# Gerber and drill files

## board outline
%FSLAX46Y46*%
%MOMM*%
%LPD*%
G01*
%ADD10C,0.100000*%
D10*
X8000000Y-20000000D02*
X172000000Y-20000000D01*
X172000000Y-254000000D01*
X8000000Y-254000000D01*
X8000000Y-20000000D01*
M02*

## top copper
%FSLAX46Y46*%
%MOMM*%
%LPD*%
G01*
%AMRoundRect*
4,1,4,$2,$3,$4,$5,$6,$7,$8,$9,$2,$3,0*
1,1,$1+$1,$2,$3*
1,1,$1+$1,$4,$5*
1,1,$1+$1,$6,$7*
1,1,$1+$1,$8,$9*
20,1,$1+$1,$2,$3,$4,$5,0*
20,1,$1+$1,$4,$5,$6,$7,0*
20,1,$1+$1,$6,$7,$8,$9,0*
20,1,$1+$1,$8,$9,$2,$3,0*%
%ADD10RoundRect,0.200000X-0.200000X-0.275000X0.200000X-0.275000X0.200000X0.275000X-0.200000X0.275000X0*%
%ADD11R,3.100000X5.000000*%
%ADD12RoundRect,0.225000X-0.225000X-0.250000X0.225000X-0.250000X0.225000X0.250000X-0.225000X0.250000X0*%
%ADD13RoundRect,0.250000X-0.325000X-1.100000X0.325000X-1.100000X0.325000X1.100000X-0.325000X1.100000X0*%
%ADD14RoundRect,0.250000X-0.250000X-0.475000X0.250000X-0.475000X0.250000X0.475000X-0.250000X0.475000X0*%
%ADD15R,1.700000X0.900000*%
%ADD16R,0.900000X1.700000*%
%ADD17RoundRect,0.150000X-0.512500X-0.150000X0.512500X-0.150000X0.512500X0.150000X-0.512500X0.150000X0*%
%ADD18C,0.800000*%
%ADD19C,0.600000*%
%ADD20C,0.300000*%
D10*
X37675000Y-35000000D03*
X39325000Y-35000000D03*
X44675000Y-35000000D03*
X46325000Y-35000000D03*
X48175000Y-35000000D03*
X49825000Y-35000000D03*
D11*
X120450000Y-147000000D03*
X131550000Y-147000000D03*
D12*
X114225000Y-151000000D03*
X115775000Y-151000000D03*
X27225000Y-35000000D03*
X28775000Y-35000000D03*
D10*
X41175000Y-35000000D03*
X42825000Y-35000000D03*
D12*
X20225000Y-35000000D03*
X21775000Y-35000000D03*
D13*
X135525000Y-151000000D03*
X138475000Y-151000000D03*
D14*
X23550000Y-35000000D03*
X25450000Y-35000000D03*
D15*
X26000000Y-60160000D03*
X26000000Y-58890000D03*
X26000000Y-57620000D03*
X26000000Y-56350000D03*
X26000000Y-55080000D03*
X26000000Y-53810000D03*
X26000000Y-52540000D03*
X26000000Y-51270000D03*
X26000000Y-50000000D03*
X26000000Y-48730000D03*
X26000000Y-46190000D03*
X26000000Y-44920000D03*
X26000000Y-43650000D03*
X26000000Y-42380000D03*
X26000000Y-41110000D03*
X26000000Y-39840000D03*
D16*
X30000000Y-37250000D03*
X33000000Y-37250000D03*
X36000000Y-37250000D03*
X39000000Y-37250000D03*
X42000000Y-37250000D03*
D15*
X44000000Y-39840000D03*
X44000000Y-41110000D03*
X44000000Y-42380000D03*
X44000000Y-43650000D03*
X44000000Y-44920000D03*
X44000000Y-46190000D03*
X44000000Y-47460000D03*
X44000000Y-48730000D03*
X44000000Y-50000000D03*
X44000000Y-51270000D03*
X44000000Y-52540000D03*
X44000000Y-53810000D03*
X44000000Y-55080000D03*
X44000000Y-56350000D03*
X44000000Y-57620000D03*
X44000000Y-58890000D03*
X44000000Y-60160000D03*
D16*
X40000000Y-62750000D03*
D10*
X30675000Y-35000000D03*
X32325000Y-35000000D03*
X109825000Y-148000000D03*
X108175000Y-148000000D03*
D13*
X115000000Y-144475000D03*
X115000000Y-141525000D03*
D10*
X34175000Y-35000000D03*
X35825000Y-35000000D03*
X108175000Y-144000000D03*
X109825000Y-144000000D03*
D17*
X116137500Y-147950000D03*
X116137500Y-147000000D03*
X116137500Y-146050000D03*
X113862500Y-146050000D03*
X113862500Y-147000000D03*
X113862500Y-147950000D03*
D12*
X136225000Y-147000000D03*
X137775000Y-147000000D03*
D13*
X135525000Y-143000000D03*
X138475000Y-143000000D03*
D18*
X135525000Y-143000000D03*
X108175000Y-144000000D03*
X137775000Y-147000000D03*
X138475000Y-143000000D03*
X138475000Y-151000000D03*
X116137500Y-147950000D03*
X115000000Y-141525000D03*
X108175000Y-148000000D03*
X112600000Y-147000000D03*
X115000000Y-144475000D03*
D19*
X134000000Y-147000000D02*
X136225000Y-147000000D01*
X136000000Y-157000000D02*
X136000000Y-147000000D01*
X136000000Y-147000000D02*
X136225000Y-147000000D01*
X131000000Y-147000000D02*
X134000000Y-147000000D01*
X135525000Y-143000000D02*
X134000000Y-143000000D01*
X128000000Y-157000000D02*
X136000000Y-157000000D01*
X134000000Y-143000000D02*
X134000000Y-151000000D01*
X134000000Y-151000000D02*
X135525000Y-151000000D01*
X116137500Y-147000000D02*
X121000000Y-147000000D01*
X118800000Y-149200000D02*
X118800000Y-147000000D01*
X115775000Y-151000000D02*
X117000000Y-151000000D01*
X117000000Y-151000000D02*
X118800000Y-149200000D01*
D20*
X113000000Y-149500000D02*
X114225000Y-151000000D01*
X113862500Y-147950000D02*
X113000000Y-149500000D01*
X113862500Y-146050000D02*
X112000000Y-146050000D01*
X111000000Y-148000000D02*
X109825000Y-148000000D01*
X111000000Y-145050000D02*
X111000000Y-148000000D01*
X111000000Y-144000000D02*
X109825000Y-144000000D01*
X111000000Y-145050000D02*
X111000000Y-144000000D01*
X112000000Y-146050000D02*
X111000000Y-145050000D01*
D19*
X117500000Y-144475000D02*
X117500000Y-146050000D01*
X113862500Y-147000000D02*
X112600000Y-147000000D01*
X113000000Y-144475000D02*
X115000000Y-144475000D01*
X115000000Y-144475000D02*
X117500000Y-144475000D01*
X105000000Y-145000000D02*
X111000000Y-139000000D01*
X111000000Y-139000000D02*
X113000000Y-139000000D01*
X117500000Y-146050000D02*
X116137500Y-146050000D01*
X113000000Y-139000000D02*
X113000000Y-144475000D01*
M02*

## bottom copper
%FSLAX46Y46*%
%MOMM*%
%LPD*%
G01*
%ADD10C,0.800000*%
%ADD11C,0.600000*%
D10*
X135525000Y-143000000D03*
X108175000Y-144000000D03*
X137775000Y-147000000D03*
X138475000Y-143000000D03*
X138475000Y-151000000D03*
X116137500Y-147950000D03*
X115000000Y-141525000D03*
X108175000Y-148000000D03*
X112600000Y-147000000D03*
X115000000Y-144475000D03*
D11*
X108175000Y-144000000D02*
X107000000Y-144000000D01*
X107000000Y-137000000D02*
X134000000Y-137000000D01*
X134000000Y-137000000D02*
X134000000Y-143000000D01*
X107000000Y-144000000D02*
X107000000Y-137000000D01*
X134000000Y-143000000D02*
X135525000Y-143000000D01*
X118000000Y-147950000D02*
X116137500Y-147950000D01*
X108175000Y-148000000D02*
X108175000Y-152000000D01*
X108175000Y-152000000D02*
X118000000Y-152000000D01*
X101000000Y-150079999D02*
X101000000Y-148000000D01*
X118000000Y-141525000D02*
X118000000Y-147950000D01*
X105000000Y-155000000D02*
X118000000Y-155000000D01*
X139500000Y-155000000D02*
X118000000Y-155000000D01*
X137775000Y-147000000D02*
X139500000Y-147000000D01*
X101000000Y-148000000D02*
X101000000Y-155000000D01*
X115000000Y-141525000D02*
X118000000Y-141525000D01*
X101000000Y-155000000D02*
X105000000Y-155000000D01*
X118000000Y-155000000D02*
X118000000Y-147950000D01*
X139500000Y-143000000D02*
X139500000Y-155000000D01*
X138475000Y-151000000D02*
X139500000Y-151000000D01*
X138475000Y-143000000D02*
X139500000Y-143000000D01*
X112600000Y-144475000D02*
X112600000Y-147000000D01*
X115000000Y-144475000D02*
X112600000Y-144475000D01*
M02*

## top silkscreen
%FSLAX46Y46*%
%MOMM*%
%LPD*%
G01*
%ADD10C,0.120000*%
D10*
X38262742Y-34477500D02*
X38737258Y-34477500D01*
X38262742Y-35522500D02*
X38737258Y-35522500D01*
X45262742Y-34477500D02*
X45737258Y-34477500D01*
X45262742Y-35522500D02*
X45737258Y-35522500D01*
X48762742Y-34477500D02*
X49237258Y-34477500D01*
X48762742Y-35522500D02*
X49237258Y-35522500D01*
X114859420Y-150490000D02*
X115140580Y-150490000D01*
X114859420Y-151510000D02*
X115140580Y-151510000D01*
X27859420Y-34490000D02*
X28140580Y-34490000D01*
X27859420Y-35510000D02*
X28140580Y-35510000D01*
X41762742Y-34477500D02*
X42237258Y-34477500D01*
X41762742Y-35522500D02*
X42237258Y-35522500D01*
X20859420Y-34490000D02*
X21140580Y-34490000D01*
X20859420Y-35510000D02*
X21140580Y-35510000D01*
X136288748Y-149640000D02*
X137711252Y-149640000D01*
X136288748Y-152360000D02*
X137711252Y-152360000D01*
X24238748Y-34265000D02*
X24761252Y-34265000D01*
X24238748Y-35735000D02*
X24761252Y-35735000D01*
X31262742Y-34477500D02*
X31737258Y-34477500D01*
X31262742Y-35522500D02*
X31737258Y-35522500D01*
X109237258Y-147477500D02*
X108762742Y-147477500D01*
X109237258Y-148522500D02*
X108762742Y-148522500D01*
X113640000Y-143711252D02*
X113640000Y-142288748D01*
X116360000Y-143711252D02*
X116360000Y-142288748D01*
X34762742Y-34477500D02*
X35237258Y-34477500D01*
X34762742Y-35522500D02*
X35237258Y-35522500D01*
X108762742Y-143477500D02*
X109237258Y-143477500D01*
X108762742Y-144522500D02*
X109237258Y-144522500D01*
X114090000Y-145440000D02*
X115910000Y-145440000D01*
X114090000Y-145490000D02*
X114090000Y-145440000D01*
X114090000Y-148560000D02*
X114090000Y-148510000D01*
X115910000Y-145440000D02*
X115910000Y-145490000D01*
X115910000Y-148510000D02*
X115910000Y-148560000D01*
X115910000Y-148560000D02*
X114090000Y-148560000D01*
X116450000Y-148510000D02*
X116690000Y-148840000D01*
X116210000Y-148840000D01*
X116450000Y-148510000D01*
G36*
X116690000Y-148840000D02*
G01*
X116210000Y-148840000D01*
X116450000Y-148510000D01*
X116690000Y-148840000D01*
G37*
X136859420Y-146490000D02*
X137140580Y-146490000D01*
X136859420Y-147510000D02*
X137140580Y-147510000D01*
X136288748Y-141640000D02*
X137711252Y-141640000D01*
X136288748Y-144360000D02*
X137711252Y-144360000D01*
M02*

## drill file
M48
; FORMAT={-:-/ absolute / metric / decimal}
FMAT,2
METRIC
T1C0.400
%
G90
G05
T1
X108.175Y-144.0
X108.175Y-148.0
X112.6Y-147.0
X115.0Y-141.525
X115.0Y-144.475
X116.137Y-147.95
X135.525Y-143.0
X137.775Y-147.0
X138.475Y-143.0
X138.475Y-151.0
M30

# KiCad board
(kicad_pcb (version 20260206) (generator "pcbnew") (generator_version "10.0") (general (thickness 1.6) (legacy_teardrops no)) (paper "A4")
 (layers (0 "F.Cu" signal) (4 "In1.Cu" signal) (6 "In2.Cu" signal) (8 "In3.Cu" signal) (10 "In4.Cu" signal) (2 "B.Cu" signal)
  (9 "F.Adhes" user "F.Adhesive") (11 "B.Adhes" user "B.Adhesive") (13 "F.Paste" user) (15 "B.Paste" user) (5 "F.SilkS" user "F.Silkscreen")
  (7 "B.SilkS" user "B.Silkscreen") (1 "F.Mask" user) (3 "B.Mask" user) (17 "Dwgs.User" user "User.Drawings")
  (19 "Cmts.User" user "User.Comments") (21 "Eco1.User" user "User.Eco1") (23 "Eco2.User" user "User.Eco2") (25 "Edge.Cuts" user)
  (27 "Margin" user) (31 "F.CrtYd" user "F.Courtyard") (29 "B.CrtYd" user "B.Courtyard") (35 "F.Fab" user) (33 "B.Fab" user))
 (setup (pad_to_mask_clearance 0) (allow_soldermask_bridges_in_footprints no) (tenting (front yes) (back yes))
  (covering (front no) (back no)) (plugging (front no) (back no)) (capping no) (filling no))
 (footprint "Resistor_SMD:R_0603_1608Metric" (layer "F.Cu") (at 38.5 35)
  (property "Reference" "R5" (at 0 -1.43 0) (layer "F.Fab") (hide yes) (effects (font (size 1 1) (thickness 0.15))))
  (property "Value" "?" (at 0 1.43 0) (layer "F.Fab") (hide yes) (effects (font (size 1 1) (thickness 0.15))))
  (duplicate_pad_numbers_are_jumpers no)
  (fp_line (start -0.237258 -0.5225) (end 0.237258 -0.5225) (stroke (width 0.12) (type solid)) (layer "F.SilkS"))
  (fp_line (start -0.237258 0.5225) (end 0.237258 0.5225) (stroke (width 0.12) (type solid)) (layer "F.SilkS"))
  (pad "1" smd roundrect (at -0.825 0) (size 0.8 0.95) (layers "F.Cu" "F.Mask" "F.Paste") (roundrect_rratio 0.25) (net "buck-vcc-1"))
  (pad "2" smd roundrect (at 0.825 0) (size 0.8 0.95) (layers "F.Cu" "F.Mask" "F.Paste") (roundrect_rratio 0.25) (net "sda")))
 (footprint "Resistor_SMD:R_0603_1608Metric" (layer "F.Cu") (at 45.5 35)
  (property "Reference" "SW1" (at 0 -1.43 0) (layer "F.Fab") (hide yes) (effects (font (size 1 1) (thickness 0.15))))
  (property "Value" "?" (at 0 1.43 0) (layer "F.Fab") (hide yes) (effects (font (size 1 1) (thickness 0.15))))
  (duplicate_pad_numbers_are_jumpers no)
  (fp_line (start -0.237258 -0.5225) (end 0.237258 -0.5225) (stroke (width 0.12) (type solid)) (layer "F.SilkS"))
  (fp_line (start -0.237258 0.5225) (end 0.237258 0.5225) (stroke (width 0.12) (type solid)) (layer "F.SilkS"))
  (pad "1" smd roundrect (at -0.825 0) (size 0.8 0.95) (layers "F.Cu" "F.Mask" "F.Paste") (roundrect_rratio 0.25) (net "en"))
  (pad "2" smd roundrect (at 0.825 0) (size 0.8 0.95) (layers "F.Cu" "F.Mask" "F.Paste") (roundrect_rratio 0.25) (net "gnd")))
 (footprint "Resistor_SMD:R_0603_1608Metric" (layer "F.Cu") (at 49 35)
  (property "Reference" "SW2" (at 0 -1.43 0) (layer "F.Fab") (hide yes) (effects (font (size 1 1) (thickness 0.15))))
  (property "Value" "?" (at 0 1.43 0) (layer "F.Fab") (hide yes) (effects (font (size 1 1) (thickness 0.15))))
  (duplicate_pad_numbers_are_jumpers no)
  (fp_line (start -0.237258 -0.5225) (end 0.237258 -0.5225) (stroke (width 0.12) (type solid)) (layer "F.SilkS"))
  (fp_line (start -0.237258 0.5225) (end 0.237258 0.5225) (stroke (width 0.12) (type solid)) (layer "F.SilkS"))
  (pad "1" smd roundrect (at -0.825 0) (size 0.8 0.95) (layers "F.Cu" "F.Mask" "F.Paste") (roundrect_rratio 0.25) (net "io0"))
  (pad "2" smd roundrect (at 0.825 0) (size 0.8 0.95) (layers "F.Cu" "F.Mask" "F.Paste") (roundrect_rratio 0.25) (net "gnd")))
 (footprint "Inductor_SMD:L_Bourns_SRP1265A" (layer "F.Cu") (at 126 147)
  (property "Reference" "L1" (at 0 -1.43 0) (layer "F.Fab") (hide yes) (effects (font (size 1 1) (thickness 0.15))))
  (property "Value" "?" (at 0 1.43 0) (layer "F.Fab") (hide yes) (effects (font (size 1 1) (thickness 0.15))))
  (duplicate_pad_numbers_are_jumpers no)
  (pad "1" smd rect (at -5.55 0) (size 3.1 5) (layers "F.Cu" "F.Mask" "F.Paste") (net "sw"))
  (pad "2" smd rect (at 5.55 0) (size 3.1 5) (layers "F.Cu" "F.Mask" "F.Paste") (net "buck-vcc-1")))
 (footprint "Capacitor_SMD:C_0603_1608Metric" (layer "F.Cu") (at 115 151)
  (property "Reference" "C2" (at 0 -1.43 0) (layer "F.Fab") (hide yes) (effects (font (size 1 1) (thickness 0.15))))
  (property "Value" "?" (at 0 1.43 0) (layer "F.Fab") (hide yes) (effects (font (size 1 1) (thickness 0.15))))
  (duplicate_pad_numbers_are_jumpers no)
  (fp_line (start -0.14058 -0.51) (end 0.14058 -0.51) (stroke (width 0.12) (type solid)) (layer "F.SilkS"))
  (fp_line (start -0.14058 0.51) (end 0.14058 0.51) (stroke (width 0.12) (type solid)) (layer "F.SilkS"))
  (pad "1" smd roundrect (at -0.775 0) (size 0.9 0.95) (layers "F.Cu" "F.Mask" "F.Paste") (roundrect_rratio 0.25) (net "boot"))
  (pad "2" smd roundrect (at 0.775 0) (size 0.9 0.95) (layers "F.Cu" "F.Mask" "F.Paste") (roundrect_rratio 0.25) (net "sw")))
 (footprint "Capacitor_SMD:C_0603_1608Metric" (layer "F.Cu") (at 28 35)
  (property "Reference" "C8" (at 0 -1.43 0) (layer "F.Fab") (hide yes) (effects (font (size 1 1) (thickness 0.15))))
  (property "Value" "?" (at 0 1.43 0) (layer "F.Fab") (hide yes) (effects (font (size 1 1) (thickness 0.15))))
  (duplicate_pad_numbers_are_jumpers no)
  (fp_line (start -0.14058 -0.51) (end 0.14058 -0.51) (stroke (width 0.12) (type solid)) (layer "F.SilkS"))
  (fp_line (start -0.14058 0.51) (end 0.14058 0.51) (stroke (width 0.12) (type solid)) (layer "F.SilkS"))
  (pad "1" smd roundrect (at -0.775 0) (size 0.9 0.95) (layers "F.Cu" "F.Mask" "F.Paste") (roundrect_rratio 0.25) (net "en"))
  (pad "2" smd roundrect (at 0.775 0) (size 0.9 0.95) (layers "F.Cu" "F.Mask" "F.Paste") (roundrect_rratio 0.25) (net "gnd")))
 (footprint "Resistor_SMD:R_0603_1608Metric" (layer "F.Cu") (at 42 35)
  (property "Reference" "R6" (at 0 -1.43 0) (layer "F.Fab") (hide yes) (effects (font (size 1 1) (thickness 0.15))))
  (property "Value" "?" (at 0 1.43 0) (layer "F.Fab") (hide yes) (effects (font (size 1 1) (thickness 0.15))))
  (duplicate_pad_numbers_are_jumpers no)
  (fp_line (start -0.237258 -0.5225) (end 0.237258 -0.5225) (stroke (width 0.12) (type solid)) (layer "F.SilkS"))
  (fp_line (start -0.237258 0.5225) (end 0.237258 0.5225) (stroke (width 0.12) (type solid)) (layer "F.SilkS"))
  (pad "1" smd roundrect (at -0.825 0) (size 0.8 0.95) (layers "F.Cu" "F.Mask" "F.Paste") (roundrect_rratio 0.25) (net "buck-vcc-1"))
  (pad "2" smd roundrect (at 0.825 0) (size 0.8 0.95) (layers "F.Cu" "F.Mask" "F.Paste") (roundrect_rratio 0.25) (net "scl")))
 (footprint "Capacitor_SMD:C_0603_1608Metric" (layer "F.Cu") (at 21 35)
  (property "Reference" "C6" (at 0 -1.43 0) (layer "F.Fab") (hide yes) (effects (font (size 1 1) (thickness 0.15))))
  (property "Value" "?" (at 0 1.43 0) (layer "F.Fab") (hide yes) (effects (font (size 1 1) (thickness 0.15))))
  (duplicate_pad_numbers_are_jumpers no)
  (fp_line (start -0.14058 -0.51) (end 0.14058 -0.51) (stroke (width 0.12) (type solid)) (layer "F.SilkS"))
  (fp_line (start -0.14058 0.51) (end 0.14058 0.51) (stroke (width 0.12) (type solid)) (layer "F.SilkS"))
  (pad "1" smd roundrect (at -0.775 0) (size 0.9 0.95) (layers "F.Cu" "F.Mask" "F.Paste") (roundrect_rratio 0.25) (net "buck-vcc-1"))
  (pad "2" smd roundrect (at 0.775 0) (size 0.9 0.95) (layers "F.Cu" "F.Mask" "F.Paste") (roundrect_rratio 0.25) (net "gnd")))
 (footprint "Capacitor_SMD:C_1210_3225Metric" (layer "F.Cu") (at 137 151)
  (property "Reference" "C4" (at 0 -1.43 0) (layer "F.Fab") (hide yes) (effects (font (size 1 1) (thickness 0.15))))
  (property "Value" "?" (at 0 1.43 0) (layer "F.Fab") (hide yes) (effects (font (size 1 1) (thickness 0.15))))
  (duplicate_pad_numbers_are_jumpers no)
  (fp_line (start -0.711252 -1.36) (end 0.711252 -1.36) (stroke (width 0.12) (type solid)) (layer "F.SilkS"))
  (fp_line (start -0.711252 1.36) (end 0.711252 1.36) (stroke (width 0.12) (type solid)) (layer "F.SilkS"))
  (pad "1" smd roundrect (at -1.475 0) (size 1.15 2.7) (layers "F.Cu" "F.Mask" "F.Paste") (roundrect_rratio 0.217391) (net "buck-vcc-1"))
  (pad "2" smd roundrect (at 1.475 0) (size 1.15 2.7) (layers "F.Cu" "F.Mask" "F.Paste") (roundrect_rratio 0.217391) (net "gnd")))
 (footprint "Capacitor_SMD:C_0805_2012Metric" (layer "F.Cu") (at 24.5 35)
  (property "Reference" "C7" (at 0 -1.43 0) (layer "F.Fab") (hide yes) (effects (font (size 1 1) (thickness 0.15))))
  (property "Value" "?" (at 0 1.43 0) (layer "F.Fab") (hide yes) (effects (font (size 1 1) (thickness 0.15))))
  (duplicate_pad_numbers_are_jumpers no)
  (fp_line (start -0.261252 -0.735) (end 0.261252 -0.735) (stroke (width 0.12) (type solid)) (layer "F.SilkS"))
  (fp_line (start -0.261252 0.735) (end 0.261252 0.735) (stroke (width 0.12) (type solid)) (layer "F.SilkS"))
  (pad "1" smd roundrect (at -0.95 0) (size 1 1.45) (layers "F.Cu" "F.Mask" "F.Paste") (roundrect_rratio 0.25) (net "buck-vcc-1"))
  (pad "2" smd roundrect (at 0.95 0) (size 1 1.45) (layers "F.Cu" "F.Mask" "F.Paste") (roundrect_rratio 0.25) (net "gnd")))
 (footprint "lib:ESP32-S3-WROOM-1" (layer "F.Cu") (at 35 50)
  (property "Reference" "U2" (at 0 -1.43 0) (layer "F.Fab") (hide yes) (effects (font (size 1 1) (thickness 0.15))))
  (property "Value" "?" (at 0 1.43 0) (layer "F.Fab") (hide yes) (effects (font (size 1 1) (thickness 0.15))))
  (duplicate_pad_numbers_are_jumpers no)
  (pad "1" smd rect (at -9 10.16) (size 1.7 0.9) (layers "F.Cu" "F.Mask" "F.Paste") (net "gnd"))
  (pad "2" smd rect (at -9 8.89) (size 1.7 0.9) (layers "F.Cu" "F.Mask" "F.Paste") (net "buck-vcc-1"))
  (pad "3" smd rect (at -9 7.62) (size 1.7 0.9) (layers "F.Cu" "F.Mask" "F.Paste") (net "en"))
  (pad "4" smd rect (at -9 6.35) (size 1.7 0.9) (layers "F.Cu" "F.Mask" "F.Paste") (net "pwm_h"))
  (pad "5" smd rect (at -9 5.08) (size 1.7 0.9) (layers "F.Cu" "F.Mask" "F.Paste") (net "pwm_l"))
  (pad "6" smd rect (at -9 3.81) (size 1.7 0.9) (layers "F.Cu" "F.Mask" "F.Paste") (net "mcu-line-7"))
  (pad "7" smd rect (at -9 2.54) (size 1.7 0.9) (layers "F.Cu" "F.Mask" "F.Paste") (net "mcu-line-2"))
  (pad "8" smd rect (at -9 1.27) (size 1.7 0.9) (layers "F.Cu" "F.Mask" "F.Paste") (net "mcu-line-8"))
  (pad "9" smd rect (at -9 0) (size 1.7 0.9) (layers "F.Cu" "F.Mask" "F.Paste") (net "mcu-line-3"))
  (pad "10" smd rect (at -9 -1.27) (size 1.7 0.9) (layers "F.Cu" "F.Mask" "F.Paste") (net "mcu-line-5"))
  (pad "11" smd rect (at -9 -3.81) (size 1.7 0.9) (layers "F.Cu" "F.Mask" "F.Paste") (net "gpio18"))
  (pad "12" smd rect (at -9 -5.08) (size 1.7 0.9) (layers "F.Cu" "F.Mask" "F.Paste") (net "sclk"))
  (pad "13" smd rect (at -9 -6.35) (size 1.7 0.9) (layers "F.Cu" "F.Mask" "F.Paste") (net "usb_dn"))
  (pad "14" smd rect (at -9 -7.62) (size 1.7 0.9) (layers "F.Cu" "F.Mask" "F.Paste") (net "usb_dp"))
  (pad "15" smd rect (at -9 -8.89) (size 1.7 0.9) (layers "F.Cu" "F.Mask" "F.Paste") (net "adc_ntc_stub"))
  (pad "16" smd rect (at -9 -10.16) (size 1.7 0.9) (layers "F.Cu" "F.Mask" "F.Paste") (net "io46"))
  (pad "17" smd rect (at -5 -12.75) (size 0.9 1.7) (layers "F.Cu" "F.Mask" "F.Paste") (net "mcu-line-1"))
  (pad "18" smd rect (at -2 -12.75) (size 0.9 1.7) (layers "F.Cu" "F.Mask" "F.Paste") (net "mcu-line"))
  (pad "19" smd rect (at 1 -12.75) (size 0.9 1.7) (layers "F.Cu" "F.Mask" "F.Paste") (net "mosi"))
  (pad "20" smd rect (at 4 -12.75) (size 0.9 1.7) (layers "F.Cu" "F.Mask" "F.Paste") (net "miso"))
  (pad "21" smd rect (at 7 -12.75) (size 0.9 1.7) (layers "F.Cu" "F.Mask" "F.Paste") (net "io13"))
  (pad "22" smd rect (at 9 -10.16) (size 1.7 0.9) (layers "F.Cu" "F.Mask" "F.Paste") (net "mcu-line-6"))
  (pad "23" smd rect (at 9 -8.89) (size 1.7 0.9) (layers "F.Cu" "F.Mask" "F.Paste") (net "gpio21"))
  (pad "24" smd rect (at 9 -7.62) (size 1.7 0.9) (layers "F.Cu" "F.Mask" "F.Paste") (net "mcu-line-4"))
  (pad "25" smd rect (at 9 -6.35) (size 1.7 0.9) (layers "F.Cu" "F.Mask" "F.Paste") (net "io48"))
  (pad "26" smd rect (at 9 -5.08) (size 1.7 0.9) (layers "F.Cu" "F.Mask" "F.Paste") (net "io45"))
  (pad "27" smd rect (at 9 -3.81) (size 1.7 0.9) (layers "F.Cu" "F.Mask" "F.Paste") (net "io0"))
  (pad "28" smd rect (at 9 -2.54) (size 1.7 0.9) (layers "F.Cu" "F.Mask" "F.Paste") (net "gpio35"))
  (pad "29" smd rect (at 9 -1.27) (size 1.7 0.9) (layers "F.Cu" "F.Mask" "F.Paste") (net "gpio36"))
  (pad "30" smd rect (at 9 0) (size 1.7 0.9) (layers "F.Cu" "F.Mask" "F.Paste") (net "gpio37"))
  (pad "31" smd rect (at 9 1.27) (size 1.7 0.9) (layers "F.Cu" "F.Mask" "F.Paste") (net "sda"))
  (pad "32" smd rect (at 9 2.54) (size 1.7 0.9) (layers "F.Cu" "F.Mask" "F.Paste") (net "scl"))
  (pad "33" smd rect (at 9 3.81) (size 1.7 0.9) (layers "F.Cu" "F.Mask" "F.Paste") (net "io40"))
  (pad "34" smd rect (at 9 5.08) (size 1.7 0.9) (layers "F.Cu" "F.Mask" "F.Paste") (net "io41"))
  (pad "35" smd rect (at 9 6.35) (size 1.7 0.9) (layers "F.Cu" "F.Mask" "F.Paste") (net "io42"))
  (pad "36" smd rect (at 9 7.62) (size 1.7 0.9) (layers "F.Cu" "F.Mask" "F.Paste") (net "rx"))
  (pad "37" smd rect (at 9 8.89) (size 1.7 0.9) (layers "F.Cu" "F.Mask" "F.Paste") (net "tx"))
  (pad "38" smd rect (at 9 10.16) (size 1.7 0.9) (layers "F.Cu" "F.Mask" "F.Paste") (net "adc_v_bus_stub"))
  (pad "39" smd rect (at 5 12.75) (size 0.9 1.7) (layers "F.Cu" "F.Mask" "F.Paste") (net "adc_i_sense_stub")))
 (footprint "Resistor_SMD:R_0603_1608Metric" (layer "F.Cu") (at 31.5 35)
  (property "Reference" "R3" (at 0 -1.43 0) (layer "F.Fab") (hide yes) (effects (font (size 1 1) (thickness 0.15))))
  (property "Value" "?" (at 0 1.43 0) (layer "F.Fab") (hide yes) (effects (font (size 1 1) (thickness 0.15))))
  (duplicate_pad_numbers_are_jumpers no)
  (fp_line (start -0.237258 -0.5225) (end 0.237258 -0.5225) (stroke (width 0.12) (type solid)) (layer "F.SilkS"))
  (fp_line (start -0.237258 0.5225) (end 0.237258 0.5225) (stroke (width 0.12) (type solid)) (layer "F.SilkS"))
  (pad "1" smd roundrect (at -0.825 0) (size 0.8 0.95) (layers "F.Cu" "F.Mask" "F.Paste") (roundrect_rratio 0.25) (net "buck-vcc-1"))
  (pad "2" smd roundrect (at 0.825 0) (size 0.8 0.95) (layers "F.Cu" "F.Mask" "F.Paste") (roundrect_rratio 0.25) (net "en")))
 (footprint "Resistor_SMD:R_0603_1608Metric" (layer "F.Cu") (at 109 148 180)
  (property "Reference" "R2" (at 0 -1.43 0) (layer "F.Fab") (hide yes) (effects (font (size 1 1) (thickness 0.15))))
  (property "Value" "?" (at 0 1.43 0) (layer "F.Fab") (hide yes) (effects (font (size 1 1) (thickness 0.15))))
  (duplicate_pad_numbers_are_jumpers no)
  (fp_line (start -0.237258 0.5225) (end 0.237258 0.5225) (stroke (width 0.12) (type solid)) (layer "F.SilkS"))
  (fp_line (start -0.237258 -0.5225) (end 0.237258 -0.5225) (stroke (width 0.12) (type solid)) (layer "F.SilkS"))
  (pad "1" smd roundrect (at -0.825 0) (size 0.8 0.95) (layers "F.Cu" "F.Mask" "F.Paste") (roundrect_rratio 0.25) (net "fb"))
  (pad "2" smd roundrect (at 0.825 0) (size 0.8 0.95) (layers "F.Cu" "F.Mask" "F.Paste") (roundrect_rratio 0.25) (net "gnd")))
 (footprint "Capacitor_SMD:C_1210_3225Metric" (layer "F.Cu") (at 115 143 90)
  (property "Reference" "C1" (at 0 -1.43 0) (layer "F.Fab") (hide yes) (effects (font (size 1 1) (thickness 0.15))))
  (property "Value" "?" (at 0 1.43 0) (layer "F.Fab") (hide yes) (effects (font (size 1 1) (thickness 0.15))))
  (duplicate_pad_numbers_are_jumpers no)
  (fp_line (start -0.711252 -1.36) (end 0.711252 -1.36) (stroke (width 0.12) (type solid)) (layer "F.SilkS"))
  (fp_line (start -0.711252 1.36) (end 0.711252 1.36) (stroke (width 0.12) (type solid)) (layer "F.SilkS"))
  (pad "1" smd roundrect (at -1.475 0) (size 1.15 2.7) (layers "F.Cu" "F.Mask" "F.Paste") (roundrect_rratio 0.217391) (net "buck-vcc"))
  (pad "2" smd roundrect (at 1.475 0) (size 1.15 2.7) (layers "F.Cu" "F.Mask" "F.Paste") (roundrect_rratio 0.217391) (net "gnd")))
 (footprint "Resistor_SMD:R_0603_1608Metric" (layer "F.Cu") (at 35 35)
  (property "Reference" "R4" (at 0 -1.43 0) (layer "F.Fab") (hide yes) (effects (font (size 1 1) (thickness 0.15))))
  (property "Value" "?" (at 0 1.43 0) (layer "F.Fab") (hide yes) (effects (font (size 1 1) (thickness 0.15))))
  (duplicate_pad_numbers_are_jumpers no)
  (fp_line (start -0.237258 -0.5225) (end 0.237258 -0.5225) (stroke (width 0.12) (type solid)) (layer "F.SilkS"))
  (fp_line (start -0.237258 0.5225) (end 0.237258 0.5225) (stroke (width 0.12) (type solid)) (layer "F.SilkS"))
  (pad "1" smd roundrect (at -0.825 0) (size 0.8 0.95) (layers "F.Cu" "F.Mask" "F.Paste") (roundrect_rratio 0.25) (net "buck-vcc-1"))
  (pad "2" smd roundrect (at 0.825 0) (size 0.8 0.95) (layers "F.Cu" "F.Mask" "F.Paste") (roundrect_rratio 0.25) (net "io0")))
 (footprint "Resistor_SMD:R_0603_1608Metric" (layer "F.Cu") (at 109 144)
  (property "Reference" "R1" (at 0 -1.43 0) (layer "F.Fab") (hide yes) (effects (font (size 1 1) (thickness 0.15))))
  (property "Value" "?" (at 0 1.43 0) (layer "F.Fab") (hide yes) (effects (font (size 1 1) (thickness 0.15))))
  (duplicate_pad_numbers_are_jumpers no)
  (fp_line (start -0.237258 -0.5225) (end 0.237258 -0.5225) (stroke (width 0.12) (type solid)) (layer "F.SilkS"))
  (fp_line (start -0.237258 0.5225) (end 0.237258 0.5225) (stroke (width 0.12) (type solid)) (layer "F.SilkS"))
  (pad "1" smd roundrect (at -0.825 0) (size 0.8 0.95) (layers "F.Cu" "F.Mask" "F.Paste") (roundrect_rratio 0.25) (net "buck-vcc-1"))
  (pad "2" smd roundrect (at 0.825 0) (size 0.8 0.95) (layers "F.Cu" "F.Mask" "F.Paste") (roundrect_rratio 0.25) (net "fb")))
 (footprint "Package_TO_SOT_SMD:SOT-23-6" (layer "F.Cu") (at 115 147 180)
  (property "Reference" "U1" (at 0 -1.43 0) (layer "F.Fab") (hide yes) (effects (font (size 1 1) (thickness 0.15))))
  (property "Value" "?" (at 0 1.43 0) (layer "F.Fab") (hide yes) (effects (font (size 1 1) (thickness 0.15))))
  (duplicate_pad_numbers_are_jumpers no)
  (fp_line (start 0.91 1.56) (end -0.91 1.56) (stroke (width 0.12) (type solid)) (layer "F.SilkS"))
  (fp_line (start 0.91 1.51) (end 0.91 1.56) (stroke (width 0.12) (type solid)) (layer "F.SilkS"))
  (fp_line (start 0.91 -1.56) (end 0.91 -1.51) (stroke (width 0.12) (type solid)) (layer "F.SilkS"))
  (fp_line (start -0.91 1.56) (end -0.91 1.51) (stroke (width 0.12) (type solid)) (layer "F.SilkS"))
  (fp_line (start -0.91 -1.51) (end -0.91 -1.56) (stroke (width 0.12) (type solid)) (layer "F.SilkS"))
  (fp_line (start -0.91 -1.56) (end 0.91 -1.56) (stroke (width 0.12) (type solid)) (layer "F.SilkS"))
  (fp_poly (pts (xy -1.45 -1.51) (xy -1.69 -1.84) (xy -1.21 -1.84)) (stroke (width 0.12) (type solid)) (fill yes) (layer "F.SilkS"))
  (pad "1" smd roundrect (at -1.1375 -0.95) (size 1.325 0.6) (layers "F.Cu" "F.Mask" "F.Paste") (roundrect_rratio 0.25) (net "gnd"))
  (pad "2" smd roundrect (at -1.1375 0) (size 1.325 0.6) (layers "F.Cu" "F.Mask" "F.Paste") (roundrect_rratio 0.25) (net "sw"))
  (pad "3" smd roundrect (at -1.1375 0.95) (size 1.325 0.6) (layers "F.Cu" "F.Mask" "F.Paste") (roundrect_rratio 0.25) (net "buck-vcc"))
  (pad "4" smd roundrect (at 1.1375 0.95) (size 1.325 0.6) (layers "F.Cu" "F.Mask" "F.Paste") (roundrect_rratio 0.25) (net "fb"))
  (pad "5" smd roundrect (at 1.1375 0) (size 1.325 0.6) (layers "F.Cu" "F.Mask" "F.Paste") (roundrect_rratio 0.25) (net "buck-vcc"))
  (pad "6" smd roundrect (at 1.1375 -0.95) (size 1.325 0.6) (layers "F.Cu" "F.Mask" "F.Paste") (roundrect_rratio 0.25) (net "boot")))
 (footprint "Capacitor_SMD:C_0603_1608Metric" (layer "F.Cu") (at 137 147)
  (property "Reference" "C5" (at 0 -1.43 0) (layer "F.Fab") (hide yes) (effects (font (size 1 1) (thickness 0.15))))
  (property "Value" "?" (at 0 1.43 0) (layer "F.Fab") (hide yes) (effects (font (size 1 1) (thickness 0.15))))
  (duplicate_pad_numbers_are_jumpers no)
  (fp_line (start -0.14058 -0.51) (end 0.14058 -0.51) (stroke (width 0.12) (type solid)) (layer "F.SilkS"))
  (fp_line (start -0.14058 0.51) (end 0.14058 0.51) (stroke (width 0.12) (type solid)) (layer "F.SilkS"))
  (pad "1" smd roundrect (at -0.775 0) (size 0.9 0.95) (layers "F.Cu" "F.Mask" "F.Paste") (roundrect_rratio 0.25) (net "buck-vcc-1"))
  (pad "2" smd roundrect (at 0.775 0) (size 0.9 0.95) (layers "F.Cu" "F.Mask" "F.Paste") (roundrect_rratio 0.25) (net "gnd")))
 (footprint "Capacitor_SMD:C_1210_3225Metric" (layer "F.Cu") (at 137 143)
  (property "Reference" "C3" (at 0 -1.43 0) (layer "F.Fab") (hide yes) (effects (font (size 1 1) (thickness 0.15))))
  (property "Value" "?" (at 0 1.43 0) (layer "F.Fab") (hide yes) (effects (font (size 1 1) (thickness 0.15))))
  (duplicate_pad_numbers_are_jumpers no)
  (fp_line (start -0.711252 -1.36) (end 0.711252 -1.36) (stroke (width 0.12) (type solid)) (layer "F.SilkS"))
  (fp_line (start -0.711252 1.36) (end 0.711252 1.36) (stroke (width 0.12) (type solid)) (layer "F.SilkS"))
  (pad "1" smd roundrect (at -1.475 0) (size 1.15 2.7) (layers "F.Cu" "F.Mask" "F.Paste") (roundrect_rratio 0.217391) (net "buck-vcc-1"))
  (pad "2" smd roundrect (at 1.475 0) (size 1.15 2.7) (layers "F.Cu" "F.Mask" "F.Paste") (roundrect_rratio 0.217391) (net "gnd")))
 (gr_poly (pts (xy 8 20) (xy 172 20) (xy 172 254) (xy 8 254)) (stroke (width 0.1) (type solid)) (fill no) (layer "Edge.Cuts"))
 (segment (start 134 147) (end 136.225 147) (width 0.6) (layer "F.Cu") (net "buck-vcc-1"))
 (segment (start 136 157) (end 136 147) (width 0.6) (layer "F.Cu") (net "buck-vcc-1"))
 (segment (start 136 147) (end 136.225 147) (width 0.6) (layer "F.Cu") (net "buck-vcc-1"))
 (segment (start 131 147) (end 134 147) (width 0.6) (layer "F.Cu") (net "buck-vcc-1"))
 (segment (start 135.525 143) (end 134 143) (width 0.6) (layer "F.Cu") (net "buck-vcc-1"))
 (segment (start 128 157) (end 136 157) (width 0.6) (layer "F.Cu") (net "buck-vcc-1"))
 (segment (start 134 143) (end 134 151) (width 0.6) (layer "F.Cu") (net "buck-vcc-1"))
 (segment (start 134 151) (end 135.525 151) (width 0.6) (layer "F.Cu") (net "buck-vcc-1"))
 (via (at 135.525 143) (size 0.8) (drill 0.4) (layers "F.Cu" "B.Cu") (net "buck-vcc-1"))
 (via (at 108.175 144) (size 0.8) (drill 0.4) (layers "F.Cu" "B.Cu") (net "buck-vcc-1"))
 (segment (start 108.175 144) (end 107 144) (width 0.6) (layer "B.Cu") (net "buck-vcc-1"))
 (segment (start 107 137) (end 134 137) (width 0.6) (layer "B.Cu") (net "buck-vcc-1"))
 (segment (start 134 137) (end 134 143) (width 0.6) (layer "B.Cu") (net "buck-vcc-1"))
 (segment (start 107 144) (end 107 137) (width 0.6) (layer "B.Cu") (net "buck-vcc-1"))
 (segment (start 134 143) (end 135.525 143) (width 0.6) (layer "B.Cu") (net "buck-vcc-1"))
 (via (at 137.775 147) (size 0.8) (drill 0.4) (layers "F.Cu" "B.Cu") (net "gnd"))
 (via (at 138.475 143) (size 0.8) (drill 0.4) (layers "F.Cu" "B.Cu") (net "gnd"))
 (via (at 138.475 151) (size 0.8) (drill 0.4) (layers "F.Cu" "B.Cu") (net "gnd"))
 (via (at 116.1375 147.95) (size 0.8) (drill 0.4) (layers "F.Cu" "B.Cu") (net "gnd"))
 (via (at 115 141.525) (size 0.8) (drill 0.4) (layers "F.Cu" "B.Cu") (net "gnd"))
 (via (at 108.175 148) (size 0.8) (drill 0.4) (layers "F.Cu" "B.Cu") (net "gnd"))
 (segment (start 118 147.95) (end 116.1375 147.95) (width 0.6) (layer "B.Cu") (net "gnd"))
 (segment (start 108.175 148) (end 108.175 152) (width 0.6) (layer "B.Cu") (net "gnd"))
 (segment (start 108.175 152) (end 118 152) (width 0.6) (layer "B.Cu") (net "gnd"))
 (segment (start 101 150.079999) (end 101 148) (width 0.6) (layer "B.Cu") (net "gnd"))
 (segment (start 118 141.525) (end 118 147.95) (width 0.6) (layer "B.Cu") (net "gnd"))
 (segment (start 105 155) (end 118 155) (width 0.6) (layer "B.Cu") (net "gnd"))
 (segment (start 139.5 155) (end 118 155) (width 0.6) (layer "B.Cu") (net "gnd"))
 (segment (start 137.775 147) (end 139.5 147) (width 0.6) (layer "B.Cu") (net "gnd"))
 (segment (start 101 148) (end 101 155) (width 0.6) (layer "B.Cu") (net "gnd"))
 (segment (start 115 141.525) (end 118 141.525) (width 0.6) (layer "B.Cu") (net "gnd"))
 (segment (start 101 155) (end 105 155) (width 0.6) (layer "B.Cu") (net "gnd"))
 (segment (start 118 155) (end 118 147.95) (width 0.6) (layer "B.Cu") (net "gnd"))
 (segment (start 139.5 143) (end 139.5 155) (width 0.6) (layer "B.Cu") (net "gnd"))
 (segment (start 138.475 151) (end 139.5 151) (width 0.6) (layer "B.Cu") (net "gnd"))
 (segment (start 138.475 143) (end 139.5 143) (width 0.6) (layer "B.Cu") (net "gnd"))
 (segment (start 116.1375 147) (end 121 147) (width 0.6) (layer "F.Cu") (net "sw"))
 (segment (start 118.8 149.2) (end 118.8 147) (width 0.6) (layer "F.Cu") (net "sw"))
 (segment (start 115.775 151) (end 117 151) (width 0.6) (layer "F.Cu") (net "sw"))
 (segment (start 117 151) (end 118.8 149.2) (width 0.6) (layer "F.Cu") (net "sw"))
 (segment (start 113 149.5) (end 114.225 151) (width 0.3) (layer "F.Cu") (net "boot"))
 (segment (start 113.8625 147.95) (end 113 149.5) (width 0.3) (layer "F.Cu") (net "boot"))
 (segment (start 113.8625 146.05) (end 112 146.05) (width 0.3) (layer "F.Cu") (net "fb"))
 (segment (start 111 148) (end 109.825 148) (width 0.3) (layer "F.Cu") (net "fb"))
 (segment (start 111 145.05) (end 111 148) (width 0.3) (layer "F.Cu") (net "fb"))
 (segment (start 111 144) (end 109.825 144) (width 0.3) (layer "F.Cu") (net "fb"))
 (segment (start 111 145.05) (end 111 144) (width 0.3) (layer "F.Cu") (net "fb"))
 (segment (start 112 146.05) (end 111 145.05) (width 0.3) (layer "F.Cu") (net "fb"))
 (segment (start 117.5 144.475) (end 117.5 146.05) (width 0.6) (layer "F.Cu") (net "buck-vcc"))
 (segment (start 113.8625 147) (end 112.6 147) (width 0.6) (layer "F.Cu") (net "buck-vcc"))
 (segment (start 113 144.475) (end 115 144.475) (width 0.6) (layer "F.Cu") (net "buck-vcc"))
 (segment (start 115 144.475) (end 117.5 144.475) (width 0.6) (layer "F.Cu") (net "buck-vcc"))
 (segment (start 105 145) (end 111 139) (width 0.6) (layer "F.Cu") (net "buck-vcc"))
 (segment (start 111 139) (end 113 139) (width 0.6) (layer "F.Cu") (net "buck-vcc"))
 (segment (start 117.5 146.05) (end 116.1375 146.05) (width 0.6) (layer "F.Cu") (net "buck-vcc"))
 (segment (start 113 139) (end 113 144.475) (width 0.6) (layer "F.Cu") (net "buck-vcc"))
 (via (at 112.6 147) (size 0.8) (drill 0.4) (layers "F.Cu" "B.Cu") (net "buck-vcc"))
 (via (at 115 144.475) (size 0.8) (drill 0.4) (layers "F.Cu" "B.Cu") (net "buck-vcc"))
 (segment (start 112.6 144.475) (end 112.6 147) (width 0.6) (layer "B.Cu") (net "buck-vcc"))
 (segment (start 115 144.475) (end 112.6 144.475) (width 0.6) (layer "B.Cu") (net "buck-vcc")))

